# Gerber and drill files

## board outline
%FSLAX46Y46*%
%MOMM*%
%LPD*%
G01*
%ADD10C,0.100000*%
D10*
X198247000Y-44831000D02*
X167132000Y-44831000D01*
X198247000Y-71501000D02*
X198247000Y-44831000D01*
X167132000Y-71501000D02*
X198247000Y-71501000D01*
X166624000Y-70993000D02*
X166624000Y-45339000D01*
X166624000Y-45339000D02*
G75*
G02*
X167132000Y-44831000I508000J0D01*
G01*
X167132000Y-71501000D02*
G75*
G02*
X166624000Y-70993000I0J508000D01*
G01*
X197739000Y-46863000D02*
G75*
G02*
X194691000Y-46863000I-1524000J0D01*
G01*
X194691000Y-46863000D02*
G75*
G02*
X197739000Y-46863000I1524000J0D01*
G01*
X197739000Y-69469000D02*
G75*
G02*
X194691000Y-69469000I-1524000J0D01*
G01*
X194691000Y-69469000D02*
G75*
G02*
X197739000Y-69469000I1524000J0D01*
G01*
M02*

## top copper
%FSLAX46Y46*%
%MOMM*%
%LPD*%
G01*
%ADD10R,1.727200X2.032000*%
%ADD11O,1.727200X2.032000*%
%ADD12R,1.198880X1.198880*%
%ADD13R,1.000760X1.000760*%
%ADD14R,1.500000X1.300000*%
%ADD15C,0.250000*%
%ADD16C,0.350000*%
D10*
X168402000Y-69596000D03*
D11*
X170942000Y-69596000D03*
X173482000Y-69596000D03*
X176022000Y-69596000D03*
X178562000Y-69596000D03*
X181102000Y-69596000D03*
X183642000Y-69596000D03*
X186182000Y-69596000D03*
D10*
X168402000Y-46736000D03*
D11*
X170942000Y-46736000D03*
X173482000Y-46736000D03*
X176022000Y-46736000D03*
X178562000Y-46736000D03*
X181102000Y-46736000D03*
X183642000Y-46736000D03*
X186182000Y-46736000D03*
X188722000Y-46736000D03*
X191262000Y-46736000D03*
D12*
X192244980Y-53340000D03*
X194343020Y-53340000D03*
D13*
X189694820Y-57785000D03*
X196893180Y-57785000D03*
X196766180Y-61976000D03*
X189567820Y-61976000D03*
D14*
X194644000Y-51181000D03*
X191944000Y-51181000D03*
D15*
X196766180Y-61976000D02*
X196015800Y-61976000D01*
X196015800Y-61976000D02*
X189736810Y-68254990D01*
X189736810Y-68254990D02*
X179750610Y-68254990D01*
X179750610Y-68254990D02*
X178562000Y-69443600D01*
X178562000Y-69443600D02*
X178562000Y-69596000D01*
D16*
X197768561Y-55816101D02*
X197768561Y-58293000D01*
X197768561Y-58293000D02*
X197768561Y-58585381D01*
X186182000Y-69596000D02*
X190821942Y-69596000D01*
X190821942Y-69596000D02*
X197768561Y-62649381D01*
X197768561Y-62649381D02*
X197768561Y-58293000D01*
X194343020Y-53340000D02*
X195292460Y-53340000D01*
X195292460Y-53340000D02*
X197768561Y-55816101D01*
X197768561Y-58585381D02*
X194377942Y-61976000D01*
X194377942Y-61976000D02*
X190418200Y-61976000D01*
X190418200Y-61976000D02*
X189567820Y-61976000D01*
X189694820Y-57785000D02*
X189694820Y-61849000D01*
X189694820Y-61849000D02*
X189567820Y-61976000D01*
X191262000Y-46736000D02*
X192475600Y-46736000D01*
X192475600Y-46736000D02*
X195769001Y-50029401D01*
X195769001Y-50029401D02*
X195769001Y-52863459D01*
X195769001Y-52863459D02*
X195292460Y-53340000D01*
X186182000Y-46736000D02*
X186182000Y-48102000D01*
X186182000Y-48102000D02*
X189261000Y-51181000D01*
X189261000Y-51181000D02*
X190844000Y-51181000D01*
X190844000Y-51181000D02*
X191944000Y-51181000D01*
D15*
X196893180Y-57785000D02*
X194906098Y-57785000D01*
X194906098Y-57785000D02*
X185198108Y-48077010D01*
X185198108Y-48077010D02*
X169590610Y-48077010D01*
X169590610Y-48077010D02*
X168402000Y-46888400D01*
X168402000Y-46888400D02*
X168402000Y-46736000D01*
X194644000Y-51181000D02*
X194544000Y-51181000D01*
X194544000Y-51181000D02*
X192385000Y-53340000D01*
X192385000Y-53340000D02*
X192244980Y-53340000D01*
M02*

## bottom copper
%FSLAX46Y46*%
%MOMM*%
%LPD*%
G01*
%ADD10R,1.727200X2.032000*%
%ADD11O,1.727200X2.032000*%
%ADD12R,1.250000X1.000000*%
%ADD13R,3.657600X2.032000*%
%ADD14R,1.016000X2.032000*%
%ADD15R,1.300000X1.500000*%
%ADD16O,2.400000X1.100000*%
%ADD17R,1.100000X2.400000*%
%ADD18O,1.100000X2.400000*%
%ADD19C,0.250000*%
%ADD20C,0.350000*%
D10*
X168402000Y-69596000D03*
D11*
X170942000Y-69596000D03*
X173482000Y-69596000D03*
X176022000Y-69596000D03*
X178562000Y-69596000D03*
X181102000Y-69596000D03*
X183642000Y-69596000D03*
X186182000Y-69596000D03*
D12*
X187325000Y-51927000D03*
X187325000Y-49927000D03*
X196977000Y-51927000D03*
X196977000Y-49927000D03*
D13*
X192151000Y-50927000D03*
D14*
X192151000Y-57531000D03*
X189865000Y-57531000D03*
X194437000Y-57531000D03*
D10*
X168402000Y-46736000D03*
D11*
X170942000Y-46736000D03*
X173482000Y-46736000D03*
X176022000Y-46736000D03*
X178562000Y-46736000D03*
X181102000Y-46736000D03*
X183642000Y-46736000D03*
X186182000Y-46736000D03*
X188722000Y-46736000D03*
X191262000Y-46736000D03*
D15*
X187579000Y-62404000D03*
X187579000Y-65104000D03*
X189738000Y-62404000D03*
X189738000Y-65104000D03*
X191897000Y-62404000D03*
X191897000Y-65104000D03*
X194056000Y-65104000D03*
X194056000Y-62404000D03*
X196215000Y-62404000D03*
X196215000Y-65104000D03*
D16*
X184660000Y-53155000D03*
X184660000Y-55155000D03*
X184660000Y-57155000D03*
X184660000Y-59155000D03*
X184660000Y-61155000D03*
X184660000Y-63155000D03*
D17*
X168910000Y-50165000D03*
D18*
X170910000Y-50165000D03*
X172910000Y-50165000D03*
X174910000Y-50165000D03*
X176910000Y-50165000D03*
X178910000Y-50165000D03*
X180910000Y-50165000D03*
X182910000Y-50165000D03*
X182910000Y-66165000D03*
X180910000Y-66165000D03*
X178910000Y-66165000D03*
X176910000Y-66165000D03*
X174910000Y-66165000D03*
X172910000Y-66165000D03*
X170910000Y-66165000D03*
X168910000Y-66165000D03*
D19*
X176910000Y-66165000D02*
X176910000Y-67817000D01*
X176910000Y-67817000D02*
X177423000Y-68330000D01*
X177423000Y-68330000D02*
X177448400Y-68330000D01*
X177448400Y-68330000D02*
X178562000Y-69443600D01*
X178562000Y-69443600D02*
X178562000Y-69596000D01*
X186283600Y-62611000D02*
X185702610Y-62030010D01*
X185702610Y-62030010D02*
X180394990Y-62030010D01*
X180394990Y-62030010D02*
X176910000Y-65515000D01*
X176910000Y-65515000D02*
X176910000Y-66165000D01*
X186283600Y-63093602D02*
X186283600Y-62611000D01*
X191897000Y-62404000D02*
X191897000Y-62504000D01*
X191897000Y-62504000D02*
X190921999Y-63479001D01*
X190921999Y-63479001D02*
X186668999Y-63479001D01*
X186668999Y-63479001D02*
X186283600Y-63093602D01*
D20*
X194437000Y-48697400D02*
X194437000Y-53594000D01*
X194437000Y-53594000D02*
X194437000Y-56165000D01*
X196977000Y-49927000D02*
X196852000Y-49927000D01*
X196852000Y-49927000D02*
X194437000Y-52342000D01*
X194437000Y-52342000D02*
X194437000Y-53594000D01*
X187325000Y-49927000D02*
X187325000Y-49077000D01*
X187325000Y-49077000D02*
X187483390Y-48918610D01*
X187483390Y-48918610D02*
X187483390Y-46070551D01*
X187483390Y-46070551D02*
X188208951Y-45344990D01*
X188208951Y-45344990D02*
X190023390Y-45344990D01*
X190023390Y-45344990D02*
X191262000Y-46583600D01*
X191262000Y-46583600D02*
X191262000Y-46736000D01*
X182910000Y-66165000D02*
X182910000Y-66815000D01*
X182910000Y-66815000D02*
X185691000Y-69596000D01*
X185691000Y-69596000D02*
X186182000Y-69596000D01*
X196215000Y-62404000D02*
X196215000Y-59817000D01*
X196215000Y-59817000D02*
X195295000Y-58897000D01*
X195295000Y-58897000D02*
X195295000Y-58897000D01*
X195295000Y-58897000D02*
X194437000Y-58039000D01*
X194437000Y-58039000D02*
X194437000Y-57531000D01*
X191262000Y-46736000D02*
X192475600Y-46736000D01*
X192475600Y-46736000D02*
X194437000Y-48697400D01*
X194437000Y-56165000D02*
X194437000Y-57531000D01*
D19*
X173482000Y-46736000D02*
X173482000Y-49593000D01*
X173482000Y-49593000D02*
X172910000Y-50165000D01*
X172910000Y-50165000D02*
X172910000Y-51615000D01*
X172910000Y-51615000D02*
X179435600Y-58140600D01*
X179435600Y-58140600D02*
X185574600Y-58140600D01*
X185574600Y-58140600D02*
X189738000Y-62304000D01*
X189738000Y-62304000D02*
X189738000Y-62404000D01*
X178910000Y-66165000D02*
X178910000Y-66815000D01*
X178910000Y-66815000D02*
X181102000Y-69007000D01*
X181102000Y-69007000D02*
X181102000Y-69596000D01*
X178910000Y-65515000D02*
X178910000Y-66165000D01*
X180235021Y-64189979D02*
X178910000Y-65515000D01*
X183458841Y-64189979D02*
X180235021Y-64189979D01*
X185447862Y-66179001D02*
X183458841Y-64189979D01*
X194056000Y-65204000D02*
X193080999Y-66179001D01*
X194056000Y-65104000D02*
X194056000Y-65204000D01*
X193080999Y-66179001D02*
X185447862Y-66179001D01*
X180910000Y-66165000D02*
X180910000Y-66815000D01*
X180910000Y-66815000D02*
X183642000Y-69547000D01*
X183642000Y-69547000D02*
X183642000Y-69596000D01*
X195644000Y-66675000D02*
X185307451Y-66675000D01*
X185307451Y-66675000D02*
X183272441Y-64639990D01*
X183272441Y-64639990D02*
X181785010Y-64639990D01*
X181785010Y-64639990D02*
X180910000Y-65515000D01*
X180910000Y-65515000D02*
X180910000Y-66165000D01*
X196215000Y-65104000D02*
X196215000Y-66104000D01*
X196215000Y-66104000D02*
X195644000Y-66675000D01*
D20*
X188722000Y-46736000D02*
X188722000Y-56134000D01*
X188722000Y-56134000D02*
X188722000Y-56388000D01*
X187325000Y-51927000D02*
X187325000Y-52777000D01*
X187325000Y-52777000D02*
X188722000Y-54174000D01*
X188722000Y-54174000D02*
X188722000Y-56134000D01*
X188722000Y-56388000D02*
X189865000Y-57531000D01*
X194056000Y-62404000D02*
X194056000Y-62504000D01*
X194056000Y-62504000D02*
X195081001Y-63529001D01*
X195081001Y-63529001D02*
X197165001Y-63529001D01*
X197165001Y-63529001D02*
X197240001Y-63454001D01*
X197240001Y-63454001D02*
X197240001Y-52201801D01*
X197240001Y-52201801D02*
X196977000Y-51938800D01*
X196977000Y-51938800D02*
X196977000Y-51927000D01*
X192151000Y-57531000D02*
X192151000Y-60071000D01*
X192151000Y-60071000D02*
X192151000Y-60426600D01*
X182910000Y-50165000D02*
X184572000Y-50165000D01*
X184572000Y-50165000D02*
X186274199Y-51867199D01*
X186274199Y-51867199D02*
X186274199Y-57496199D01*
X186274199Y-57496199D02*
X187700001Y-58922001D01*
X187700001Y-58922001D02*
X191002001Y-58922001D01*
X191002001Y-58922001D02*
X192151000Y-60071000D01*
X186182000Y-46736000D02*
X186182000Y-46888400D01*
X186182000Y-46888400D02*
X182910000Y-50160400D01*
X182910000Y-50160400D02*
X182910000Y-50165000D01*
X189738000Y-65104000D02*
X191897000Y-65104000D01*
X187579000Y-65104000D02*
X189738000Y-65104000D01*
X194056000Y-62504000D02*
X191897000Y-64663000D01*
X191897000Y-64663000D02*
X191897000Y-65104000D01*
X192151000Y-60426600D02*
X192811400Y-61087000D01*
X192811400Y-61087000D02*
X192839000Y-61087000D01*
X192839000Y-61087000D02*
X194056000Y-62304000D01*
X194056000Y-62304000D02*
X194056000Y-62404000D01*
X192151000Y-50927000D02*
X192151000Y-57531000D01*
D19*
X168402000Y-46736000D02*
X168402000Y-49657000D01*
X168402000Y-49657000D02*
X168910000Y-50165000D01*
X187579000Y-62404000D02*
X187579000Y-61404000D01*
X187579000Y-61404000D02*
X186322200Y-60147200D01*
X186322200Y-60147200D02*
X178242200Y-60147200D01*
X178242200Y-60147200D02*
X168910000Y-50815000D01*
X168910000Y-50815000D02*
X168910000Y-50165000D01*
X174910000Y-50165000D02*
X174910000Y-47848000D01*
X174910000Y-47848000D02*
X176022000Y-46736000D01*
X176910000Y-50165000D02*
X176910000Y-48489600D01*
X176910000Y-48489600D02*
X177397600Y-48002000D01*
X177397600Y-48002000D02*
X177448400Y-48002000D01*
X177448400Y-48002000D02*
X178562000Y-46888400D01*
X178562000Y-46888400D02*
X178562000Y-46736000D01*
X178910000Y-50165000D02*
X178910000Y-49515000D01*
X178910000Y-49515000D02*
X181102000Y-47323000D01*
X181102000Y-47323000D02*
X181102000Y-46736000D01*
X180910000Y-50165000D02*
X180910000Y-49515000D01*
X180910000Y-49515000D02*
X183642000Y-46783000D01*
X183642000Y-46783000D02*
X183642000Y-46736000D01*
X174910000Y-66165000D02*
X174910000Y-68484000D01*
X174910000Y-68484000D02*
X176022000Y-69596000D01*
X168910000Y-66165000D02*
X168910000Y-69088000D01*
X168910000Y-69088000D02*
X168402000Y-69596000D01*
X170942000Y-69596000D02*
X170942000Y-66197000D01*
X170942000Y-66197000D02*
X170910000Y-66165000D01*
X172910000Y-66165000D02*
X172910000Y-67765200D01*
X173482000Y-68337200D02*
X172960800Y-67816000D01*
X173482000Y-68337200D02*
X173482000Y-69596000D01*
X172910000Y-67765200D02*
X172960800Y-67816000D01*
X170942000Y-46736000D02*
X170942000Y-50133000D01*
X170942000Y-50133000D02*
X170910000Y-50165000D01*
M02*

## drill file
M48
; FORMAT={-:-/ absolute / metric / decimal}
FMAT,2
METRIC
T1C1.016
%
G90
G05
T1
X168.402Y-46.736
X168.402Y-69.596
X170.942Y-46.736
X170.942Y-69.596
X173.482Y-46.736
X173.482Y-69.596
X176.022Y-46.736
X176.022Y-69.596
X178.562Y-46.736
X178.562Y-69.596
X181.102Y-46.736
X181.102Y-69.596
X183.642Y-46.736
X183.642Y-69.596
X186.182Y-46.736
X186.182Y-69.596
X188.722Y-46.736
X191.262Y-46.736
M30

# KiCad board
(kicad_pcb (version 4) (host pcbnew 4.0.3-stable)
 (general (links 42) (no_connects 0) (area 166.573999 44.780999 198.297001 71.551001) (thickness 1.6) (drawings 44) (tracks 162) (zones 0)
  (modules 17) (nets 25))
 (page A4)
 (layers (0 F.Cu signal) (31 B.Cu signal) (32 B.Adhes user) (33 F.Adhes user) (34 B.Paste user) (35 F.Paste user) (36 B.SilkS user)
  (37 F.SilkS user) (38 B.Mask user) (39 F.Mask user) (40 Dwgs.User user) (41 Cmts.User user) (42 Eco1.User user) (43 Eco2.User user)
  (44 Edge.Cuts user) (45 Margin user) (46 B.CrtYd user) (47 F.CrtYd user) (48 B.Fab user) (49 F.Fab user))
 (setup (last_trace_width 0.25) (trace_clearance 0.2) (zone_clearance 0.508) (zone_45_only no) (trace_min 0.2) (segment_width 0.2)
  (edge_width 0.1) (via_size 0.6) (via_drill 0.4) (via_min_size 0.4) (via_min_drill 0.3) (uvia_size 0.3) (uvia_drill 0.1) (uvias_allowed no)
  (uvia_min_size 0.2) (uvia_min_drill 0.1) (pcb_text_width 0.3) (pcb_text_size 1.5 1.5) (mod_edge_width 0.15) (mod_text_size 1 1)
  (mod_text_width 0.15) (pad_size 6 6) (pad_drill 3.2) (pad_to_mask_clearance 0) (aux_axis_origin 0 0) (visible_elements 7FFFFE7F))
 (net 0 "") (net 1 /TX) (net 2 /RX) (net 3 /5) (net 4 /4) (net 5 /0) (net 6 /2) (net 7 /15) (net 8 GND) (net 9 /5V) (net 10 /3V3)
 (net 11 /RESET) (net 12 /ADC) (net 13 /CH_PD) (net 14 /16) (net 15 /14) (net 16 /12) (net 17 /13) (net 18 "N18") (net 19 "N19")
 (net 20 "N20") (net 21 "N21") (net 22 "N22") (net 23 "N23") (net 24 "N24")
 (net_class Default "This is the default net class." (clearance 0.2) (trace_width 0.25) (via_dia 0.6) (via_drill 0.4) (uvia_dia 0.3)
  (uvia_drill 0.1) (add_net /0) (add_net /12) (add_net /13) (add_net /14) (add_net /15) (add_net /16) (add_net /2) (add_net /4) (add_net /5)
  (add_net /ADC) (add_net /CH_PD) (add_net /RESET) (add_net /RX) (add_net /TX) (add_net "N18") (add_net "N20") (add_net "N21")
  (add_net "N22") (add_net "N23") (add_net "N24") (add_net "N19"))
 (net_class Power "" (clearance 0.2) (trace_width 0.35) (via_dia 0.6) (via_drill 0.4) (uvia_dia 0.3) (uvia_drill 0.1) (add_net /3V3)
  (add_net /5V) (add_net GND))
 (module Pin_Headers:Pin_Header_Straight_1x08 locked (layer B.Cu) (at 168.402 69.596 270)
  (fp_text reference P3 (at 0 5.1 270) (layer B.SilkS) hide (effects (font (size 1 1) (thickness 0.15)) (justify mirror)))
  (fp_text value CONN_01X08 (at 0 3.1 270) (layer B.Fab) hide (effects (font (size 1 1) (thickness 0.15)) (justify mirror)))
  (pad 1 thru_hole rect (at 0 0 270) (size 2.032 1.7272) (drill 1.016) (layers *.Cu *.Mask B.SilkS) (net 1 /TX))
  (pad 2 thru_hole oval (at 0 -2.54 270) (size 2.032 1.7272) (drill 1.016) (layers *.Cu *.Mask B.SilkS) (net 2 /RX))
  (pad 3 thru_hole oval (at 0 -5.08 270) (size 2.032 1.7272) (drill 1.016) (layers *.Cu *.Mask B.SilkS) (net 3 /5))
  (pad 4 thru_hole oval (at 0 -7.62 270) (size 2.032 1.7272) (drill 1.016) (layers *.Cu *.Mask B.SilkS) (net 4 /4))
  (pad 5 thru_hole oval (at 0 -10.16 270) (size 2.032 1.7272) (drill 1.016) (layers *.Cu *.Mask B.SilkS) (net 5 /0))
  (pad 6 thru_hole oval (at 0 -12.7 270) (size 2.032 1.7272) (drill 1.016) (layers *.Cu *.Mask B.SilkS) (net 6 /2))
  (pad 7 thru_hole oval (at 0 -15.24 270) (size 2.032 1.7272) (drill 1.016) (layers *.Cu *.Mask B.SilkS) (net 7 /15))
  (pad 8 thru_hole oval (at 0 -17.78 270) (size 2.032 1.7272) (drill 1.016) (layers *.Cu *.Mask B.SilkS) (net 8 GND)))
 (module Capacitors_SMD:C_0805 (layer B.Cu) (at 187.325 50.927 90)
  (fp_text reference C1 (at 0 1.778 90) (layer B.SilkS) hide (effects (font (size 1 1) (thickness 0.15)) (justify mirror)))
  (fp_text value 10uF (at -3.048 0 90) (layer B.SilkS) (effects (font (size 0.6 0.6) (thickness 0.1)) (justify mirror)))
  (pad 1 smd rect (at -1 0 90) (size 1 1.25) (layers B.Cu B.Paste B.Mask) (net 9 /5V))
  (pad 2 smd rect (at 1 0 90) (size 1 1.25) (layers B.Cu B.Paste B.Mask) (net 8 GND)))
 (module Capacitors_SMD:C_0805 (layer B.Cu) (at 196.977 50.927 90)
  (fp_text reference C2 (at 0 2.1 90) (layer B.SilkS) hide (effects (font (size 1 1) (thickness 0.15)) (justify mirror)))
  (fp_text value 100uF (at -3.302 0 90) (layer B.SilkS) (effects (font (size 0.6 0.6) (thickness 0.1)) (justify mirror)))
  (pad 1 smd rect (at -1 0 90) (size 1 1.25) (layers B.Cu B.Paste B.Mask) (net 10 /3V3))
  (pad 2 smd rect (at 1 0 90) (size 1 1.25) (layers B.Cu B.Paste B.Mask) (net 8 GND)))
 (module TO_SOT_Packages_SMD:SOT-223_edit (layer B.Cu) (at 192.151 54.229 180)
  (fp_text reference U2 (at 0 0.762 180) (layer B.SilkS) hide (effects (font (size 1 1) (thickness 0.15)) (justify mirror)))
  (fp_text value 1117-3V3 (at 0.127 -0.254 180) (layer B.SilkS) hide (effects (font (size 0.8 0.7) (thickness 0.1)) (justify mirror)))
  (pad 2 smd rect (at 0 3.302 180) (size 3.6576 2.032) (layers B.Cu B.Paste B.Mask) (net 10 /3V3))
  (pad 2 smd rect (at 0 -3.302 180) (size 1.016 2.032) (layers B.Cu B.Paste B.Mask) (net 10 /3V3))
  (pad 3 smd rect (at 2.286 -3.302 180) (size 1.016 2.032) (layers B.Cu B.Paste B.Mask) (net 9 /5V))
  (pad 1 smd rect (at -2.286 -3.302 180) (size 1.016 2.032) (layers B.Cu B.Paste B.Mask) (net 8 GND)))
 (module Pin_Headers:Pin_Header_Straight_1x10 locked (layer B.Cu) (at 168.402 46.736 270)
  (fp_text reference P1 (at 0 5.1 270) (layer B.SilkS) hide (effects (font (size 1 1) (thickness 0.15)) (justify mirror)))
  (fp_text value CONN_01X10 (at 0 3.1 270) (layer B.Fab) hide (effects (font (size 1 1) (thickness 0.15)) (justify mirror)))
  (pad 1 thru_hole rect (at 0 0 270) (size 2.032 1.7272) (drill 1.016) (layers *.Cu *.Mask B.SilkS) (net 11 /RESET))
  (pad 2 thru_hole oval (at 0 -2.54 270) (size 2.032 1.7272) (drill 1.016) (layers *.Cu *.Mask B.SilkS) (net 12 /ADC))
  (pad 3 thru_hole oval (at 0 -5.08 270) (size 2.032 1.7272) (drill 1.016) (layers *.Cu *.Mask B.SilkS) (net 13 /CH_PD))
  (pad 4 thru_hole oval (at 0 -7.62 270) (size 2.032 1.7272) (drill 1.016) (layers *.Cu *.Mask B.SilkS) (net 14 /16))
  (pad 5 thru_hole oval (at 0 -10.16 270) (size 2.032 1.7272) (drill 1.016) (layers *.Cu *.Mask B.SilkS) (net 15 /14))
  (pad 6 thru_hole oval (at 0 -12.7 270) (size 2.032 1.7272) (drill 1.016) (layers *.Cu *.Mask B.SilkS) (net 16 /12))
  (pad 7 thru_hole oval (at 0 -15.24 270) (size 2.032 1.7272) (drill 1.016) (layers *.Cu *.Mask B.SilkS) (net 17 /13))
  (pad 8 thru_hole oval (at 0 -17.78 270) (size 2.032 1.7272) (drill 1.016) (layers *.Cu *.Mask B.SilkS) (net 10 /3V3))
  (pad 9 thru_hole oval (at 0 -20.32 270) (size 2.032 1.7272) (drill 1.016) (layers *.Cu *.Mask B.SilkS) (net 9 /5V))
  (pad 10 thru_hole oval (at 0 -22.86 270) (size 2.032 1.7272) (drill 1.016) (layers *.Cu *.Mask B.SilkS) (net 8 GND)))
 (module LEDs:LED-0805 (layer F.Cu) (at 193.294 53.34 180)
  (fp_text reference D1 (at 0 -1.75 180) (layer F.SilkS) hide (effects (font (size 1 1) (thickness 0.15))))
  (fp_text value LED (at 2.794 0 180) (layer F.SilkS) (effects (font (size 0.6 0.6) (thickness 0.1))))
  (pad 2 smd rect (at 1.04902 0) (size 1.19888 1.19888) (layers F.Cu F.Paste F.Mask) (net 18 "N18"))
  (pad 1 smd rect (at -1.04902 0) (size 1.19888 1.19888) (layers F.Cu F.Paste F.Mask) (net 8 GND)))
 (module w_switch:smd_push (layer F.Cu) (at 193.294 57.785) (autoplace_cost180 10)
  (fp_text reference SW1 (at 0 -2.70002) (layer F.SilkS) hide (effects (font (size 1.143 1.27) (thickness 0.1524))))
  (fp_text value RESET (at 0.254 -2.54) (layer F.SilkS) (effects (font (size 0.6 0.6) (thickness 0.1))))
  (pad 1 smd rect (at -3.59918 0) (size 1.00076 1.00076) (layers F.Cu F.Paste F.Mask) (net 8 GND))
  (pad 2 smd rect (at 3.59918 0) (size 1.00076 1.00076) (layers F.Cu F.Paste F.Mask) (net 11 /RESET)))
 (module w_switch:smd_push (layer F.Cu) (at 193.167 61.976 180) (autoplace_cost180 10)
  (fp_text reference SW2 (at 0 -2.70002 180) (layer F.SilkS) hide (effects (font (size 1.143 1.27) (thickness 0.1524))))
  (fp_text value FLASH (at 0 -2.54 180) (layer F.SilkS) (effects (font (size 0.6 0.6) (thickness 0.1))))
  (pad 1 smd rect (at -3.59918 0 180) (size 1.00076 1.00076) (layers F.Cu F.Paste F.Mask) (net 5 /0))
  (pad 2 smd rect (at 3.59918 0 180) (size 1.00076 1.00076) (layers F.Cu F.Paste F.Mask) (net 8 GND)))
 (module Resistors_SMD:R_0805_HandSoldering (layer B.Cu) (at 187.579 63.754 270)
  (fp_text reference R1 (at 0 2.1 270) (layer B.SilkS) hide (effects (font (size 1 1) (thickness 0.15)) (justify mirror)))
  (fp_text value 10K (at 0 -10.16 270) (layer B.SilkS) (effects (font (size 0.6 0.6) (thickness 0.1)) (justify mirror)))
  (pad 1 smd rect (at -1.35 0 270) (size 1.5 1.3) (layers B.Cu B.Paste B.Mask) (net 11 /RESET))
  (pad 2 smd rect (at 1.35 0 270) (size 1.5 1.3) (layers B.Cu B.Paste B.Mask) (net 10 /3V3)))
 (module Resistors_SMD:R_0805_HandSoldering (layer B.Cu) (at 189.738 63.754 270)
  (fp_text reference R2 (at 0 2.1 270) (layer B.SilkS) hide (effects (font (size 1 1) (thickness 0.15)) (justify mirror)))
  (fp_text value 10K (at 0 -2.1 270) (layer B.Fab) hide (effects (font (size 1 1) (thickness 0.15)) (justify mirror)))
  (pad 1 smd rect (at -1.35 0 270) (size 1.5 1.3) (layers B.Cu B.Paste B.Mask) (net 13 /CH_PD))
  (pad 2 smd rect (at 1.35 0 270) (size 1.5 1.3) (layers B.Cu B.Paste B.Mask) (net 10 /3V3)))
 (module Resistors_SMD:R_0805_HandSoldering (layer B.Cu) (at 191.897 63.754 270)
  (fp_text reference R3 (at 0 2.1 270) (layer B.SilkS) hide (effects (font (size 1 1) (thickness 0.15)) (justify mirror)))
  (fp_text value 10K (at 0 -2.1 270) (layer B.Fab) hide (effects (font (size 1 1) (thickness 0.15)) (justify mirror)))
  (pad 1 smd rect (at -1.35 0 270) (size 1.5 1.3) (layers B.Cu B.Paste B.Mask) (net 5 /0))
  (pad 2 smd rect (at 1.35 0 270) (size 1.5 1.3) (layers B.Cu B.Paste B.Mask) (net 10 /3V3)))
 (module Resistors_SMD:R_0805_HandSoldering (layer B.Cu) (at 194.056 63.754 90)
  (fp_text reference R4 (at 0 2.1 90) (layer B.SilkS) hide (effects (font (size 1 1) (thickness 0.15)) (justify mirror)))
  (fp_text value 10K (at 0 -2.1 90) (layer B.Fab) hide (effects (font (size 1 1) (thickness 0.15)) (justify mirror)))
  (pad 1 smd rect (at -1.35 0 90) (size 1.5 1.3) (layers B.Cu B.Paste B.Mask) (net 6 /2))
  (pad 2 smd rect (at 1.35 0 90) (size 1.5 1.3) (layers B.Cu B.Paste B.Mask) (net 10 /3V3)))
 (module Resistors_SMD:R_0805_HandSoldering (layer B.Cu) (at 196.215 63.754 270)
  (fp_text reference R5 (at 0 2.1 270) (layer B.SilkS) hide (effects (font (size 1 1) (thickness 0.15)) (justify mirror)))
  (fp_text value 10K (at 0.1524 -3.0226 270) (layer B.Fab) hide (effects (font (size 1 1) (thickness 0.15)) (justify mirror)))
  (pad 1 smd rect (at -1.35 0 270) (size 1.5 1.3) (layers B.Cu B.Paste B.Mask) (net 8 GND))
  (pad 2 smd rect (at 1.35 0 270) (size 1.5 1.3) (layers B.Cu B.Paste B.Mask) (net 7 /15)))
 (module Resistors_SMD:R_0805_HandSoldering (layer F.Cu) (at 193.294 51.181 180)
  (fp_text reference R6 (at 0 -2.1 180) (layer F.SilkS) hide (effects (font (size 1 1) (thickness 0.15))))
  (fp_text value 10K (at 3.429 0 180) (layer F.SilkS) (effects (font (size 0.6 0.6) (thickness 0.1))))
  (pad 1 smd rect (at -1.35 0 180) (size 1.5 1.3) (layers F.Cu F.Paste F.Mask) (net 18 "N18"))
  (pad 2 smd rect (at 1.35 0 180) (size 1.5 1.3) (layers F.Cu F.Paste F.Mask) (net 10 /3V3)))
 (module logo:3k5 (layer F.Cu) (at 177.546 56.515)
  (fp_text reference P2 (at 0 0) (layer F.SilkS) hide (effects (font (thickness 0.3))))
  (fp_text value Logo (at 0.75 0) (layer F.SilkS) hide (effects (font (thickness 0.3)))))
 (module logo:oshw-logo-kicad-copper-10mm (layer F.Cu) (at 190.627 67.564)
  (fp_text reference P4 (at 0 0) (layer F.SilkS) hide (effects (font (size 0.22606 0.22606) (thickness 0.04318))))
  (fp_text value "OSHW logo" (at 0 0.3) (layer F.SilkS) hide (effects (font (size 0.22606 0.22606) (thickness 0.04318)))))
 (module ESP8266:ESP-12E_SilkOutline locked (layer B.Cu) (at 168.91 50.165 270)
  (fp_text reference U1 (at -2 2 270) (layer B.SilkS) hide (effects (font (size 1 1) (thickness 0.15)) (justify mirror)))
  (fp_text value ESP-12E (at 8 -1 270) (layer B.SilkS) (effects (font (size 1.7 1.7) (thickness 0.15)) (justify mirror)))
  (pad 9 smd oval (at 2.99 -15.75 180) (size 2.4 1.1) (layers B.Cu B.Paste B.Mask) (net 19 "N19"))
  (pad 10 smd oval (at 4.99 -15.75 180) (size 2.4 1.1) (layers B.Cu B.Paste B.Mask) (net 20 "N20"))
  (pad 11 smd oval (at 6.99 -15.75 180) (size 2.4 1.1) (layers B.Cu B.Paste B.Mask) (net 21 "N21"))
  (pad 12 smd oval (at 8.99 -15.75 180) (size 2.4 1.1) (layers B.Cu B.Paste B.Mask) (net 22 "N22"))
  (pad 13 smd oval (at 10.99 -15.75 180) (size 2.4 1.1) (layers B.Cu B.Paste B.Mask) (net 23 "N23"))
  (pad 14 smd oval (at 12.99 -15.75 180) (size 2.4 1.1) (layers B.Cu B.Paste B.Mask) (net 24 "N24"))
  (pad 1 smd rect (at 0 0 270) (size 2.4 1.1) (layers B.Cu B.Paste B.Mask) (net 11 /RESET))
  (pad 2 smd oval (at 0 -2 270) (size 2.4 1.1) (layers B.Cu B.Paste B.Mask) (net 12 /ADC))
  (pad 3 smd oval (at 0 -4 270) (size 2.4 1.1) (layers B.Cu B.Paste B.Mask) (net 13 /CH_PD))
  (pad 4 smd oval (at 0 -6 270) (size 2.4 1.1) (layers B.Cu B.Paste B.Mask) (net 14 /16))
  (pad 5 smd oval (at 0 -8 270) (size 2.4 1.1) (layers B.Cu B.Paste B.Mask) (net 15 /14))
  (pad 6 smd oval (at 0 -10 270) (size 2.4 1.1) (layers B.Cu B.Paste B.Mask) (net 16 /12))
  (pad 7 smd oval (at 0 -12 270) (size 2.4 1.1) (layers B.Cu B.Paste B.Mask) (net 17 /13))
  (pad 8 smd oval (at 0 -14 270) (size 2.4 1.1) (layers B.Cu B.Paste B.Mask) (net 10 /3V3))
  (pad 15 smd oval (at 16 -14 270) (size 2.4 1.1) (layers B.Cu B.Paste B.Mask) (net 8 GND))
  (pad 16 smd oval (at 16 -12 270) (size 2.4 1.1) (layers B.Cu B.Paste B.Mask) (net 7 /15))
  (pad 17 smd oval (at 16 -10 270) (size 2.4 1.1) (layers B.Cu B.Paste B.Mask) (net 6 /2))
  (pad 18 smd oval (at 16 -8 270) (size 2.4 1.1) (layers B.Cu B.Paste B.Mask) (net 5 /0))
  (pad 19 smd oval (at 16 -6 270) (size 2.4 1.1) (layers B.Cu B.Paste B.Mask) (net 4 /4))
  (pad 20 smd oval (at 16 -4 270) (size 2.4 1.1) (layers B.Cu B.Paste B.Mask) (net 3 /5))
  (pad 21 smd oval (at 16 -2 270) (size 2.4 1.1) (layers B.Cu B.Paste B.Mask) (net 2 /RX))
  (pad 22 smd oval (at 16 0 270) (size 2.4 1.1) (layers B.Cu B.Paste B.Mask) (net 1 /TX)))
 (gr_line (start 198.247 44.831) (end 167.132 44.831) (angle 90) (layer Edge.Cuts) (width 0.1))
 (gr_line (start 198.247 71.501) (end 198.247 44.831) (angle 90) (layer Edge.Cuts) (width 0.1))
 (gr_line (start 167.132 71.501) (end 198.247 71.501) (angle 90) (layer Edge.Cuts) (width 0.1))
 (gr_line (start 166.624 70.993) (end 166.624 45.339) (angle 90) (layer Edge.Cuts) (width 0.1))
 (gr_arc (start 167.132 45.339) (end 166.624 45.339) (angle 90) (layer Edge.Cuts) (width 0.1))
 (gr_arc (start 167.132 70.993) (end 167.132 71.501) (angle 90) (layer Edge.Cuts) (width 0.1))
 (gr_circle (center 196.215 46.863) (end 196.215 45.339) (layer Edge.Cuts) (width 0.1))
 (gr_circle (center 196.215 69.469) (end 196.215 67.945) (layer Edge.Cuts) (width 0.1))
 (segment (start 196.76618 61.976) (end 196.0158 61.976) (width 0.25) (layer F.Cu) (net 5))
 (segment (start 196.0158 61.976) (end 189.73681 68.25499) (width 0.25) (layer F.Cu) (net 5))
 (segment (start 189.73681 68.25499) (end 179.75061 68.25499) (width 0.25) (layer F.Cu) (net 5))
 (segment (start 179.75061 68.25499) (end 178.562 69.4436) (width 0.25) (layer F.Cu) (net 5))
 (segment (start 178.562 69.4436) (end 178.562 69.596) (width 0.25) (layer F.Cu) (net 5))
 (segment (start 176.91 66.165) (end 176.91 67.817) (width 0.25) (layer B.Cu) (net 5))
 (segment (start 176.91 67.817) (end 177.423 68.33) (width 0.25) (layer B.Cu) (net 5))
 (segment (start 177.423 68.33) (end 177.4484 68.33) (width 0.25) (layer B.Cu) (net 5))
 (segment (start 177.4484 68.33) (end 178.562 69.4436) (width 0.25) (layer B.Cu) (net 5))
 (segment (start 178.562 69.4436) (end 178.562 69.596) (width 0.25) (layer B.Cu) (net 5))
 (segment (start 186.2836 62.611) (end 185.70261 62.03001) (width 0.25) (layer B.Cu) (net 5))
 (segment (start 185.70261 62.03001) (end 180.39499 62.03001) (width 0.25) (layer B.Cu) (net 5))
 (segment (start 180.39499 62.03001) (end 176.91 65.515) (width 0.25) (layer B.Cu) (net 5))
 (segment (start 176.91 65.515) (end 176.91 66.165) (width 0.25) (layer B.Cu) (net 5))
 (segment (start 186.2836 63.093602) (end 186.2836 62.611) (width 0.25) (layer B.Cu) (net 5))
 (segment (start 191.897 62.404) (end 191.897 62.504) (width 0.25) (layer B.Cu) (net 5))
 (segment (start 191.897 62.504) (end 190.921999 63.479001) (width 0.25) (layer B.Cu) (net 5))
 (segment (start 190.921999 63.479001) (end 186.668999 63.479001) (width 0.25) (layer B.Cu) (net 5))
 (segment (start 186.668999 63.479001) (end 186.2836 63.093602) (width 0.25) (layer B.Cu) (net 5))
 (segment (start 194.437 48.6974) (end 194.437 53.594) (width 0.35) (layer B.Cu) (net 8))
 (segment (start 194.437 53.594) (end 194.437 56.165) (width 0.35) (layer B.Cu) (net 8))
 (segment (start 196.977 49.927) (end 196.852 49.927) (width 0.35) (layer B.Cu) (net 8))
 (segment (start 196.852 49.927) (end 194.437 52.342) (width 0.35) (layer B.Cu) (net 8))
 (segment (start 194.437 52.342) (end 194.437 53.594) (width 0.35) (layer B.Cu) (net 8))
 (segment (start 197.768561 55.816101) (end 197.768561 58.293) (width 0.35) (layer F.Cu) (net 8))
 (segment (start 197.768561 58.293) (end 197.768561 58.585381) (width 0.35) (layer F.Cu) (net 8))
 (segment (start 186.182 69.596) (end 190.821942 69.596) (width 0.35) (layer F.Cu) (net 8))
 (segment (start 190.821942 69.596) (end 197.768561 62.649381) (width 0.35) (layer F.Cu) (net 8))
 (segment (start 197.768561 62.649381) (end 197.768561 58.293) (width 0.35) (layer F.Cu) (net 8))
 (segment (start 187.325 49.927) (end 187.325 49.077) (width 0.35) (layer B.Cu) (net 8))
 (segment (start 187.325 49.077) (end 187.48339 48.91861) (width 0.35) (layer B.Cu) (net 8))
 (segment (start 187.48339 48.91861) (end 187.48339 46.070551) (width 0.35) (layer B.Cu) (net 8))
 (segment (start 187.48339 46.070551) (end 188.208951 45.34499) (width 0.35) (layer B.Cu) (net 8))
 (segment (start 188.208951 45.34499) (end 190.02339 45.34499) (width 0.35) (layer B.Cu) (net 8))
 (segment (start 190.02339 45.34499) (end 191.262 46.5836) (width 0.35) (layer B.Cu) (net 8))
 (segment (start 191.262 46.5836) (end 191.262 46.736) (width 0.35) (layer B.Cu) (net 8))
 (segment (start 194.34302 53.34) (end 195.29246 53.34) (width 0.35) (layer F.Cu) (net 8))
 (segment (start 195.29246 53.34) (end 197.768561 55.816101) (width 0.35) (layer F.Cu) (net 8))
 (segment (start 197.768561 58.585381) (end 194.377942 61.976) (width 0.35) (layer F.Cu) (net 8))
 (segment (start 194.377942 61.976) (end 190.4182 61.976) (width 0.35) (layer F.Cu) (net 8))
 (segment (start 190.4182 61.976) (end 189.56782 61.976) (width 0.35) (layer F.Cu) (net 8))
 (segment (start 189.69482 57.785) (end 189.69482 61.849) (width 0.35) (layer F.Cu) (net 8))
 (segment (start 189.69482 61.849) (end 189.56782 61.976) (width 0.35) (layer F.Cu) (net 8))
 (segment (start 191.262 46.736) (end 192.4756 46.736) (width 0.35) (layer F.Cu) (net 8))
 (segment (start 192.4756 46.736) (end 195.769001 50.029401) (width 0.35) (layer F.Cu) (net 8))
 (segment (start 195.769001 50.029401) (end 195.769001 52.863459) (width 0.35) (layer F.Cu) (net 8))
 (segment (start 195.769001 52.863459) (end 195.29246 53.34) (width 0.35) (layer F.Cu) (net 8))
 (segment (start 182.91 66.165) (end 182.91 66.815) (width 0.35) (layer B.Cu) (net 8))
 (segment (start 182.91 66.815) (end 185.691 69.596) (width 0.35) (layer B.Cu) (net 8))
 (segment (start 185.691 69.596) (end 186.182 69.596) (width 0.35) (layer B.Cu) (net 8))
 (segment (start 196.215 62.404) (end 196.215 59.817) (width 0.35) (layer B.Cu) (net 8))
 (segment (start 196.215 59.817) (end 195.295 58.897) (width 0.35) (layer B.Cu) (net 8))
 (segment (start 195.295 58.897) (end 195.295 58.897) (width 0.35) (layer B.Cu) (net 8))
 (segment (start 195.295 58.897) (end 194.437 58.039) (width 0.35) (layer B.Cu) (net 8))
 (segment (start 194.437 58.039) (end 194.437 57.531) (width 0.35) (layer B.Cu) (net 8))
 (segment (start 191.262 46.736) (end 192.4756 46.736) (width 0.35) (layer B.Cu) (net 8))
 (segment (start 192.4756 46.736) (end 194.437 48.6974) (width 0.35) (layer B.Cu) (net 8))
 (segment (start 194.437 56.165) (end 194.437 57.531) (width 0.35) (layer B.Cu) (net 8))
 (segment (start 173.482 46.736) (end 173.482 49.593) (width 0.25) (layer B.Cu) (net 13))
 (segment (start 173.482 49.593) (end 172.91 50.165) (width 0.25) (layer B.Cu) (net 13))
 (segment (start 172.91 50.165) (end 172.91 51.615) (width 0.25) (layer B.Cu) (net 13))
 (segment (start 172.91 51.615) (end 179.4356 58.1406) (width 0.25) (layer B.Cu) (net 13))
 (segment (start 179.4356 58.1406) (end 185.5746 58.1406) (width 0.25) (layer B.Cu) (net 13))
 (segment (start 185.5746 58.1406) (end 189.738 62.304) (width 0.25) (layer B.Cu) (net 13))
 (segment (start 189.738 62.304) (end 189.738 62.404) (width 0.25) (layer B.Cu) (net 13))
 (segment (start 178.91 66.165) (end 178.91 66.815) (width 0.25) (layer B.Cu) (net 6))
 (segment (start 178.91 66.815) (end 181.102 69.007) (width 0.25) (layer B.Cu) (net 6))
 (segment (start 181.102 69.007) (end 181.102 69.596) (width 0.25) (layer B.Cu) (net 6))
 (segment (start 178.91 65.515) (end 178.91 66.165) (width 0.25) (layer B.Cu) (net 6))
 (segment (start 180.235021 64.189979) (end 178.91 65.515) (width 0.25) (layer B.Cu) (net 6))
 (segment (start 183.458841 64.189979) (end 180.235021 64.189979) (width 0.25) (layer B.Cu) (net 6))
 (segment (start 185.447862 66.179001) (end 183.458841 64.189979) (width 0.25) (layer B.Cu) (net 6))
 (segment (start 194.056 65.204) (end 193.080999 66.179001) (width 0.25) (layer B.Cu) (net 6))
 (segment (start 194.056 65.104) (end 194.056 65.204) (width 0.25) (layer B.Cu) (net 6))
 (segment (start 193.080999 66.179001) (end 185.447862 66.179001) (width 0.25) (layer B.Cu) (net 6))
 (segment (start 180.91 66.165) (end 180.91 66.815) (width 0.25) (layer B.Cu) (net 7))
 (segment (start 180.91 66.815) (end 183.642 69.547) (width 0.25) (layer B.Cu) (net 7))
 (segment (start 183.642 69.547) (end 183.642 69.596) (width 0.25) (layer B.Cu) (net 7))
 (segment (start 195.644 66.675) (end 185.307451 66.675) (width 0.25) (layer B.Cu) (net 7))
 (segment (start 185.307451 66.675) (end 183.272441 64.63999) (width 0.25) (layer B.Cu) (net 7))
 (segment (start 183.272441 64.63999) (end 181.78501 64.63999) (width 0.25) (layer B.Cu) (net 7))
 (segment (start 181.78501 64.63999) (end 180.91 65.515) (width 0.25) (layer B.Cu) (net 7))
 (segment (start 180.91 65.515) (end 180.91 66.165) (width 0.25) (layer B.Cu) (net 7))
 (segment (start 196.215 65.104) (end 196.215 66.104) (width 0.25) (layer B.Cu) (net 7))
 (segment (start 196.215 66.104) (end 195.644 66.675) (width 0.25) (layer B.Cu) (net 7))
 (segment (start 188.722 46.736) (end 188.722 56.134) (width 0.35) (layer B.Cu) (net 9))
 (segment (start 188.722 56.134) (end 188.722 56.388) (width 0.35) (layer B.Cu) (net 9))
 (segment (start 187.325 51.927) (end 187.325 52.777) (width 0.35) (layer B.Cu) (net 9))
 (segment (start 187.325 52.777) (end 188.722 54.174) (width 0.35) (layer B.Cu) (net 9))
 (segment (start 188.722 54.174) (end 188.722 56.134) (width 0.35) (layer B.Cu) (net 9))
 (segment (start 188.722 56.388) (end 189.865 57.531) (width 0.35) (layer B.Cu) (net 9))
 (segment (start 194.056 62.404) (end 194.056 62.504) (width 0.35) (layer B.Cu) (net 10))
 (segment (start 194.056 62.504) (end 195.081001 63.529001) (width 0.35) (layer B.Cu) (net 10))
 (segment (start 195.081001 63.529001) (end 197.165001 63.529001) (width 0.35) (layer B.Cu) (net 10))
 (segment (start 197.165001 63.529001) (end 197.240001 63.454001) (width 0.35) (layer B.Cu) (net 10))
 (segment (start 197.240001 63.454001) (end 197.240001 52.201801) (width 0.35) (layer B.Cu) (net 10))
 (segment (start 197.240001 52.201801) (end 196.977 51.9388) (width 0.35) (layer B.Cu) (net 10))
 (segment (start 196.977 51.9388) (end 196.977 51.927) (width 0.35) (layer B.Cu) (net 10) (status 800000))
 (segment (start 192.151 57.531) (end 192.151 60.071) (width 0.35) (layer B.Cu) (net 10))
 (segment (start 192.151 60.071) (end 192.151 60.4266) (width 0.35) (layer B.Cu) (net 10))
 (segment (start 182.91 50.165) (end 184.572 50.165) (width 0.35) (layer B.Cu) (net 10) (status 400000))
 (segment (start 184.572 50.165) (end 186.274199 51.867199) (width 0.35) (layer B.Cu) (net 10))
 (segment (start 186.274199 51.867199) (end 186.274199 57.496199) (width 0.35) (layer B.Cu) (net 10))
 (segment (start 186.274199 57.496199) (end 187.700001 58.922001) (width 0.35) (layer B.Cu) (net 10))
 (segment (start 187.700001 58.922001) (end 191.002001 58.922001) (width 0.35) (layer B.Cu) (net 10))
 (segment (start 191.002001 58.922001) (end 192.151 60.071) (width 0.35) (layer B.Cu) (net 10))
 (segment (start 186.182 46.736) (end 186.182 48.102) (width 0.35) (layer F.Cu) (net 10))
 (segment (start 186.182 48.102) (end 189.261 51.181) (width 0.35) (layer F.Cu) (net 10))
 (segment (start 189.261 51.181) (end 190.844 51.181) (width 0.35) (layer F.Cu) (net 10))
 (segment (start 190.844 51.181) (end 191.944 51.181) (width 0.35) (layer F.Cu) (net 10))
 (segment (start 186.182 46.736) (end 186.182 46.8884) (width 0.35) (layer B.Cu) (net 10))
 (segment (start 186.182 46.8884) (end 182.91 50.1604) (width 0.35) (layer B.Cu) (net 10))
 (segment (start 182.91 50.1604) (end 182.91 50.165) (width 0.35) (layer B.Cu) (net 10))
 (segment (start 189.738 65.104) (end 191.897 65.104) (width 0.35) (layer B.Cu) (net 10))
 (segment (start 187.579 65.104) (end 189.738 65.104) (width 0.35) (layer B.Cu) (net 10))
 (segment (start 194.056 62.504) (end 191.897 64.663) (width 0.35) (layer B.Cu) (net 10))
 (segment (start 191.897 64.663) (end 191.897 65.104) (width 0.35) (layer B.Cu) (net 10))
 (segment (start 192.151 60.4266) (end 192.8114 61.087) (width 0.35) (layer B.Cu) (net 10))
 (segment (start 192.8114 61.087) (end 192.839 61.087) (width 0.35) (layer B.Cu) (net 10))
 (segment (start 192.839 61.087) (end 194.056 62.304) (width 0.35) (layer B.Cu) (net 10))
 (segment (start 194.056 62.304) (end 194.056 62.404) (width 0.35) (layer B.Cu) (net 10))
 (segment (start 192.151 50.927) (end 192.151 57.531) (width 0.35) (layer B.Cu) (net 10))
 (segment (start 196.89318 57.785) (end 194.906098 57.785) (width 0.25) (layer F.Cu) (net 11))
 (segment (start 194.906098 57.785) (end 185.198108 48.07701) (width 0.25) (layer F.Cu) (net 11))
 (segment (start 185.198108 48.07701) (end 169.59061 48.07701) (width 0.25) (layer F.Cu) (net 11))
 (segment (start 169.59061 48.07701) (end 168.402 46.8884) (width 0.25) (layer F.Cu) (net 11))
 (segment (start 168.402 46.8884) (end 168.402 46.736) (width 0.25) (layer F.Cu) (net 11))
 (segment (start 168.402 46.736) (end 168.402 49.657) (width 0.25) (layer B.Cu) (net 11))
 (segment (start 168.402 49.657) (end 168.91 50.165) (width 0.25) (layer B.Cu) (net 11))
 (segment (start 187.579 62.404) (end 187.579 61.404) (width 0.25) (layer B.Cu) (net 11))
 (segment (start 187.579 61.404) (end 186.3222 60.1472) (width 0.25) (layer B.Cu) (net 11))
 (segment (start 186.3222 60.1472) (end 178.2422 60.1472) (width 0.25) (layer B.Cu) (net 11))
 (segment (start 178.2422 60.1472) (end 168.91 50.815) (width 0.25) (layer B.Cu) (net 11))
 (segment (start 168.91 50.815) (end 168.91 50.165) (width 0.25) (layer B.Cu) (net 11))
 (segment (start 174.91 50.165) (end 174.91 47.848) (width 0.25) (layer B.Cu) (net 14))
 (segment (start 174.91 47.848) (end 176.022 46.736) (width 0.25) (layer B.Cu) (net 14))
 (segment (start 176.91 50.165) (end 176.91 48.4896) (width 0.25) (layer B.Cu) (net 15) (status 400000))
 (segment (start 176.91 48.4896) (end 177.3976 48.002) (width 0.25) (layer B.Cu) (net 15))
 (segment (start 177.3976 48.002) (end 177.4484 48.002) (width 0.25) (layer B.Cu) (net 15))
 (segment (start 177.4484 48.002) (end 178.562 46.8884) (width 0.25) (layer B.Cu) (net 15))
 (segment (start 178.562 46.8884) (end 178.562 46.736) (width 0.25) (layer B.Cu) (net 15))
 (segment (start 178.91 50.165) (end 178.91 49.515) (width 0.25) (layer B.Cu) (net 16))
 (segment (start 178.91 49.515) (end 181.102 47.323) (width 0.25) (layer B.Cu) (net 16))
 (segment (start 181.102 47.323) (end 181.102 46.736) (width 0.25) (layer B.Cu) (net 16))
 (segment (start 180.91 50.165) (end 180.91 49.515) (width 0.25) (layer B.Cu) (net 17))
 (segment (start 180.91 49.515) (end 183.642 46.783) (width 0.25) (layer B.Cu) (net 17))
 (segment (start 183.642 46.783) (end 183.642 46.736) (width 0.25) (layer B.Cu) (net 17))
 (segment (start 174.91 66.165) (end 174.91 68.484) (width 0.25) (layer B.Cu) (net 4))
 (segment (start 174.91 68.484) (end 176.022 69.596) (width 0.25) (layer B.Cu) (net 4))
 (segment (start 168.91 66.165) (end 168.91 69.088) (width 0.25) (layer B.Cu) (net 1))
 (segment (start 168.91 69.088) (end 168.402 69.596) (width 0.25) (layer B.Cu) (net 1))
 (segment (start 170.942 69.596) (end 170.942 66.197) (width 0.25) (layer B.Cu) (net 2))
 (segment (start 170.942 66.197) (end 170.91 66.165) (width 0.25) (layer B.Cu) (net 2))
 (segment (start 172.91 66.165) (end 172.91 67.7652) (width 0.25) (layer B.Cu) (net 3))
 (segment (start 173.482 68.3372) (end 172.9608 67.816) (width 0.25) (layer B.Cu) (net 3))
 (segment (start 173.482 68.3372) (end 173.482 69.596) (width 0.25) (layer B.Cu) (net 3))
 (segment (start 172.91 67.7652) (end 172.9608 67.816) (width 0.25) (layer B.Cu) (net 3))
 (segment (start 170.942 46.736) (end 170.942 50.133) (width 0.25) (layer B.Cu) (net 12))
 (segment (start 170.942 50.133) (end 170.91 50.165) (width 0.25) (layer B.Cu) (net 12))
 (segment (start 194.644 51.181) (end 194.544 51.181) (width 0.25) (layer F.Cu) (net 18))
 (segment (start 194.544 51.181) (end 192.385 53.34) (width 0.25) (layer F.Cu) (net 18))
 (segment (start 192.385 53.34) (end 192.24498 53.34) (width 0.25) (layer F.Cu) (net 18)))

